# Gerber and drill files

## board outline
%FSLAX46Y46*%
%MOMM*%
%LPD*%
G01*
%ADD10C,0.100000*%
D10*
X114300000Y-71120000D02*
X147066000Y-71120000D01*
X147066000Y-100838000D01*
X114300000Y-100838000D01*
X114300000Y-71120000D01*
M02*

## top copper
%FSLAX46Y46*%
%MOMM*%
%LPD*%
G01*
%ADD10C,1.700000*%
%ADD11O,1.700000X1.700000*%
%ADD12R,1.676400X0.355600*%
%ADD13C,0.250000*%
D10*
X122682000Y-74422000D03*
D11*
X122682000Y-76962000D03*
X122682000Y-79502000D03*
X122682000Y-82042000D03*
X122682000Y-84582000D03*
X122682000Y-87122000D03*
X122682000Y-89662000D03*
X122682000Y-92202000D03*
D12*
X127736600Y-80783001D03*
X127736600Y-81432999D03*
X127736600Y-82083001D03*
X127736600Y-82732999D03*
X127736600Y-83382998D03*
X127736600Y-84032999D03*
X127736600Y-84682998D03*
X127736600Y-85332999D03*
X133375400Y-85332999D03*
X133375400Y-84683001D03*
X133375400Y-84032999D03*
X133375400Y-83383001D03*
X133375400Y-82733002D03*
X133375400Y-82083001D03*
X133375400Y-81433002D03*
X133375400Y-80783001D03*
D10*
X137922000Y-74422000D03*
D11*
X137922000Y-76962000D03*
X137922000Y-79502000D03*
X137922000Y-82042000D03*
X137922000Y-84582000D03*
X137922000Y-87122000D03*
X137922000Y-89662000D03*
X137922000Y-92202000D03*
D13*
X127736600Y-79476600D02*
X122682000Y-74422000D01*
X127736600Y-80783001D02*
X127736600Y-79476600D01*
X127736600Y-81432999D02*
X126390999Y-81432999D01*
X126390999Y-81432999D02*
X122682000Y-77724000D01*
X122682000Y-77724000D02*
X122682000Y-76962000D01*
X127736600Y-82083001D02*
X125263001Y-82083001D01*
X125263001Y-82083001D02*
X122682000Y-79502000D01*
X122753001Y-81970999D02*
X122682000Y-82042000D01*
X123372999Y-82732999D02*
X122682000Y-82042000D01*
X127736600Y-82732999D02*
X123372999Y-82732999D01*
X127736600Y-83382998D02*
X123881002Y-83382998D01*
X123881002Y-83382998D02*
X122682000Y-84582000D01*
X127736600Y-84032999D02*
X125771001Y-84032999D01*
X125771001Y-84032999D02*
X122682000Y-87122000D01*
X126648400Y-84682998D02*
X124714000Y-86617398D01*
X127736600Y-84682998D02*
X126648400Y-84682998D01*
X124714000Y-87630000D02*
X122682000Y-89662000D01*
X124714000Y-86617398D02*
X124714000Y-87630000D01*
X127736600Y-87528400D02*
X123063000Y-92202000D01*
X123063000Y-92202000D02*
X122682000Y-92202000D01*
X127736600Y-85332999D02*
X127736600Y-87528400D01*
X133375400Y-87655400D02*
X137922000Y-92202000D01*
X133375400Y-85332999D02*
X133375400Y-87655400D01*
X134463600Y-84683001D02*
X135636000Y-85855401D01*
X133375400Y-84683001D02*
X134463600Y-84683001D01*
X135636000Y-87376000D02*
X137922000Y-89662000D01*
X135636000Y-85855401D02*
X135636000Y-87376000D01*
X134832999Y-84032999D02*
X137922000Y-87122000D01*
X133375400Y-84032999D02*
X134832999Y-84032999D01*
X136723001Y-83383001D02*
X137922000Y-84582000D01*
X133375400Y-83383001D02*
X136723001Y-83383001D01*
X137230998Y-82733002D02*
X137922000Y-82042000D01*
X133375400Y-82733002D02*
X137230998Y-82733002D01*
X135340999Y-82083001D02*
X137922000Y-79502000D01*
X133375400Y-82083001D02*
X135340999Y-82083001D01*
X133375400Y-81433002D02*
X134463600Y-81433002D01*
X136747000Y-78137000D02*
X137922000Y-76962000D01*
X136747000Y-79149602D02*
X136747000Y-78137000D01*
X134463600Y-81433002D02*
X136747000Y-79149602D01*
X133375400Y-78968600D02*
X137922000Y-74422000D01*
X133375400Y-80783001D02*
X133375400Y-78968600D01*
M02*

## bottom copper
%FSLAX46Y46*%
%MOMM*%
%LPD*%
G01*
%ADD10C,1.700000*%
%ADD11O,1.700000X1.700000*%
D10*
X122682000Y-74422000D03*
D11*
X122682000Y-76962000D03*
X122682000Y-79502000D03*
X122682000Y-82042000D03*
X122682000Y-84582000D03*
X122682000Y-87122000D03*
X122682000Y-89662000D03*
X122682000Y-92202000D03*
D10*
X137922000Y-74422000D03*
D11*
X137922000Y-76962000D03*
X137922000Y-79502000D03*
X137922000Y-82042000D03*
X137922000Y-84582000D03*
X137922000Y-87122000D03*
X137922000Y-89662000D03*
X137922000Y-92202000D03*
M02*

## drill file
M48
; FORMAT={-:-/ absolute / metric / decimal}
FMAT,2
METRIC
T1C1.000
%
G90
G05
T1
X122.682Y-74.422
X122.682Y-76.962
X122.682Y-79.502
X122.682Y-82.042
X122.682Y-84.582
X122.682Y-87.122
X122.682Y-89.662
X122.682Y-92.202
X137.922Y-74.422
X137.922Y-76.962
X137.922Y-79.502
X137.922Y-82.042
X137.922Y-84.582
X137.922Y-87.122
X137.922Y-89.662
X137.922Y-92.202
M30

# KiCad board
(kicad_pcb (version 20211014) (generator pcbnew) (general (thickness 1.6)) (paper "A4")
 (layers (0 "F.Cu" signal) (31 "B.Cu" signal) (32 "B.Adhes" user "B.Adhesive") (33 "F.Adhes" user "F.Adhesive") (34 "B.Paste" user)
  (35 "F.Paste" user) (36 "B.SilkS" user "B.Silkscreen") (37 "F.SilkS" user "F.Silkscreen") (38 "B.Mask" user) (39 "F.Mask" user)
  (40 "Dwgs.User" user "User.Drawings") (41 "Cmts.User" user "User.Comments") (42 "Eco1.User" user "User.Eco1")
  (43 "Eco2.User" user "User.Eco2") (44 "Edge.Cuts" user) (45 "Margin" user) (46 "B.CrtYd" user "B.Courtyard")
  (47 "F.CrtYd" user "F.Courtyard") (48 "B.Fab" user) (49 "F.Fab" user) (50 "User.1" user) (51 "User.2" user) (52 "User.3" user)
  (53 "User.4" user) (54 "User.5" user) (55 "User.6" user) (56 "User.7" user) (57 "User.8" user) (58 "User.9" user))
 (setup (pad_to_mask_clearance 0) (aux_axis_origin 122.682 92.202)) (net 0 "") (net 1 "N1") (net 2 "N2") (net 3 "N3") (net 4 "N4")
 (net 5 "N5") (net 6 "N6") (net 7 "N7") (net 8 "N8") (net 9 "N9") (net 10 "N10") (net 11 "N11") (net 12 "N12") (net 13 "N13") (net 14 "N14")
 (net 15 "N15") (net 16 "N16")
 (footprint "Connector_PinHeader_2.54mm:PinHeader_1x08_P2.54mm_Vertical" (layer "F.Cu") (at 122.682 74.422)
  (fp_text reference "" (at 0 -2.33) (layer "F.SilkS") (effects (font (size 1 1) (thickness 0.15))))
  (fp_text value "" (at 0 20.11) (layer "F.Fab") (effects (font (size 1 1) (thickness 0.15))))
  (pad "1" thru_hole circle (at 0 0) (size 1.7 1.7) (drill 1) (layers *.Cu *.Mask) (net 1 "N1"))
  (pad "2" thru_hole oval (at 0 2.54) (size 1.7 1.7) (drill 1) (layers *.Cu *.Mask) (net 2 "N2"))
  (pad "3" thru_hole oval (at 0 5.08) (size 1.7 1.7) (drill 1) (layers *.Cu *.Mask) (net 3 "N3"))
  (pad "4" thru_hole oval (at 0 7.62) (size 1.7 1.7) (drill 1) (layers *.Cu *.Mask) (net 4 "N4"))
  (pad "5" thru_hole oval (at 0 10.16) (size 1.7 1.7) (drill 1) (layers *.Cu *.Mask) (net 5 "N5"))
  (pad "6" thru_hole oval (at 0 12.7) (size 1.7 1.7) (drill 1) (layers *.Cu *.Mask) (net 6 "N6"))
  (pad "7" thru_hole oval (at 0 15.24) (size 1.7 1.7) (drill 1) (layers *.Cu *.Mask) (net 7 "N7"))
  (pad "8" thru_hole oval (at 0 17.78) (size 1.7 1.7) (drill 1) (layers *.Cu *.Mask) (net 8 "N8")))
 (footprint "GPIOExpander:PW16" (layer "F.Cu") (at 130.556 83.058)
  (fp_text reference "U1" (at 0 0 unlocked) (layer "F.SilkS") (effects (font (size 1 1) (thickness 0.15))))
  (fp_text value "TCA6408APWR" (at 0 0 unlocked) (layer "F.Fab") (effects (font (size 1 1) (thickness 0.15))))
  (pad "1" smd rect (at -2.8194 -2.274999) (size 1.6764 0.3556) (layers "F.Cu" "F.Paste" "F.Mask") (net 1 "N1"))
  (pad "2" smd rect (at -2.8194 -1.625001) (size 1.6764 0.3556) (layers "F.Cu" "F.Paste" "F.Mask") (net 2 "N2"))
  (pad "3" smd rect (at -2.8194 -0.974999) (size 1.6764 0.3556) (layers "F.Cu" "F.Paste" "F.Mask") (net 3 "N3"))
  (pad "4" smd rect (at -2.8194 -0.325001) (size 1.6764 0.3556) (layers "F.Cu" "F.Paste" "F.Mask") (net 4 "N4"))
  (pad "5" smd rect (at -2.8194 0.324998) (size 1.6764 0.3556) (layers "F.Cu" "F.Paste" "F.Mask") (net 5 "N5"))
  (pad "6" smd rect (at -2.8194 0.974999) (size 1.6764 0.3556) (layers "F.Cu" "F.Paste" "F.Mask") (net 6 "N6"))
  (pad "7" smd rect (at -2.8194 1.624998) (size 1.6764 0.3556) (layers "F.Cu" "F.Paste" "F.Mask") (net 7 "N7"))
  (pad "8" smd rect (at -2.8194 2.274999) (size 1.6764 0.3556) (layers "F.Cu" "F.Paste" "F.Mask") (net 8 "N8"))
  (pad "9" smd rect (at 2.8194 2.274999) (size 1.6764 0.3556) (layers "F.Cu" "F.Paste" "F.Mask") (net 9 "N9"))
  (pad "10" smd rect (at 2.8194 1.625001) (size 1.6764 0.3556) (layers "F.Cu" "F.Paste" "F.Mask") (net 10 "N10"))
  (pad "11" smd rect (at 2.8194 0.974999) (size 1.6764 0.3556) (layers "F.Cu" "F.Paste" "F.Mask") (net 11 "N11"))
  (pad "12" smd rect (at 2.8194 0.325001) (size 1.6764 0.3556) (layers "F.Cu" "F.Paste" "F.Mask") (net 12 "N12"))
  (pad "13" smd rect (at 2.8194 -0.324998) (size 1.6764 0.3556) (layers "F.Cu" "F.Paste" "F.Mask") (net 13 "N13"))
  (pad "14" smd rect (at 2.8194 -0.974999) (size 1.6764 0.3556) (layers "F.Cu" "F.Paste" "F.Mask") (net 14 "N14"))
  (pad "15" smd rect (at 2.8194 -1.624998) (size 1.6764 0.3556) (layers "F.Cu" "F.Paste" "F.Mask") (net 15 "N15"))
  (pad "16" smd rect (at 2.8194 -2.274999) (size 1.6764 0.3556) (layers "F.Cu" "F.Paste" "F.Mask") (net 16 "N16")))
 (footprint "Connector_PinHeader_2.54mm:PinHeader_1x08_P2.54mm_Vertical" (layer "F.Cu") (at 137.922 74.422)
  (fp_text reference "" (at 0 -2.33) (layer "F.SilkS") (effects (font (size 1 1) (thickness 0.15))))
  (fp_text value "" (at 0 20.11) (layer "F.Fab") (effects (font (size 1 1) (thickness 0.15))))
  (pad "1" thru_hole circle (at 0 0) (size 1.7 1.7) (drill 1) (layers *.Cu *.Mask) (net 16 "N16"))
  (pad "2" thru_hole oval (at 0 2.54) (size 1.7 1.7) (drill 1) (layers *.Cu *.Mask) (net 15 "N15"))
  (pad "3" thru_hole oval (at 0 5.08) (size 1.7 1.7) (drill 1) (layers *.Cu *.Mask) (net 14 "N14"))
  (pad "4" thru_hole oval (at 0 7.62) (size 1.7 1.7) (drill 1) (layers *.Cu *.Mask) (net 13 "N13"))
  (pad "5" thru_hole oval (at 0 10.16) (size 1.7 1.7) (drill 1) (layers *.Cu *.Mask) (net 12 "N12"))
  (pad "6" thru_hole oval (at 0 12.7) (size 1.7 1.7) (drill 1) (layers *.Cu *.Mask) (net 11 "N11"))
  (pad "7" thru_hole oval (at 0 15.24) (size 1.7 1.7) (drill 1) (layers *.Cu *.Mask) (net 10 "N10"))
  (pad "8" thru_hole oval (at 0 17.78) (size 1.7 1.7) (drill 1) (layers *.Cu *.Mask) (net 9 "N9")))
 (gr_rect (start 114.3 71.12) (end 147.066 100.838) (layer "Edge.Cuts") (width 0.1) (fill none))
 (segment (start 127.7366 79.4766) (end 122.682 74.422) (width 0.25) (layer "F.Cu") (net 1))
 (segment (start 127.7366 80.783001) (end 127.7366 79.4766) (width 0.25) (layer "F.Cu") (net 1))
 (segment (start 127.7366 81.432999) (end 126.390999 81.432999) (width 0.25) (layer "F.Cu") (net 2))
 (segment (start 126.390999 81.432999) (end 122.682 77.724) (width 0.25) (layer "F.Cu") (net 2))
 (segment (start 122.682 77.724) (end 122.682 76.962) (width 0.25) (layer "F.Cu") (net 2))
 (segment (start 127.7366 82.083001) (end 125.263001 82.083001) (width 0.25) (layer "F.Cu") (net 3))
 (segment (start 125.263001 82.083001) (end 122.682 79.502) (width 0.25) (layer "F.Cu") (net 3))
 (segment (start 122.753001 81.970999) (end 122.682 82.042) (width 0.25) (layer "F.Cu") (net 4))
 (segment (start 123.372999 82.732999) (end 122.682 82.042) (width 0.25) (layer "F.Cu") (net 4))
 (segment (start 127.7366 82.732999) (end 123.372999 82.732999) (width 0.25) (layer "F.Cu") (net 4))
 (segment (start 127.7366 83.382998) (end 123.881002 83.382998) (width 0.25) (layer "F.Cu") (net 5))
 (segment (start 123.881002 83.382998) (end 122.682 84.582) (width 0.25) (layer "F.Cu") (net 5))
 (segment (start 127.7366 84.032999) (end 125.771001 84.032999) (width 0.25) (layer "F.Cu") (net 6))
 (segment (start 125.771001 84.032999) (end 122.682 87.122) (width 0.25) (layer "F.Cu") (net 6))
 (segment (start 126.6484 84.682998) (end 124.714 86.617398) (width 0.25) (layer "F.Cu") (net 7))
 (segment (start 127.7366 84.682998) (end 126.6484 84.682998) (width 0.25) (layer "F.Cu") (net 7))
 (segment (start 124.714 87.63) (end 122.682 89.662) (width 0.25) (layer "F.Cu") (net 7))
 (segment (start 124.714 86.617398) (end 124.714 87.63) (width 0.25) (layer "F.Cu") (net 7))
 (segment (start 127.7366 87.5284) (end 123.063 92.202) (width 0.25) (layer "F.Cu") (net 8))
 (segment (start 123.063 92.202) (end 122.682 92.202) (width 0.25) (layer "F.Cu") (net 8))
 (segment (start 127.7366 85.332999) (end 127.7366 87.5284) (width 0.25) (layer "F.Cu") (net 8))
 (segment (start 133.3754 87.6554) (end 137.922 92.202) (width 0.25) (layer "F.Cu") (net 9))
 (segment (start 133.3754 85.332999) (end 133.3754 87.6554) (width 0.25) (layer "F.Cu") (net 9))
 (segment (start 134.4636 84.683001) (end 135.636 85.855401) (width 0.25) (layer "F.Cu") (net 10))
 (segment (start 133.3754 84.683001) (end 134.4636 84.683001) (width 0.25) (layer "F.Cu") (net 10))
 (segment (start 135.636 87.376) (end 137.922 89.662) (width 0.25) (layer "F.Cu") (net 10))
 (segment (start 135.636 85.855401) (end 135.636 87.376) (width 0.25) (layer "F.Cu") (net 10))
 (segment (start 134.832999 84.032999) (end 137.922 87.122) (width 0.25) (layer "F.Cu") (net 11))
 (segment (start 133.3754 84.032999) (end 134.832999 84.032999) (width 0.25) (layer "F.Cu") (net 11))
 (segment (start 136.723001 83.383001) (end 137.922 84.582) (width 0.25) (layer "F.Cu") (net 12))
 (segment (start 133.3754 83.383001) (end 136.723001 83.383001) (width 0.25) (layer "F.Cu") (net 12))
 (segment (start 137.230998 82.733002) (end 137.922 82.042) (width 0.25) (layer "F.Cu") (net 13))
 (segment (start 133.3754 82.733002) (end 137.230998 82.733002) (width 0.25) (layer "F.Cu") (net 13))
 (segment (start 135.340999 82.083001) (end 137.922 79.502) (width 0.25) (layer "F.Cu") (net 14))
 (segment (start 133.3754 82.083001) (end 135.340999 82.083001) (width 0.25) (layer "F.Cu") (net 14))
 (segment (start 133.3754 81.433002) (end 134.4636 81.433002) (width 0.25) (layer "F.Cu") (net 15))
 (segment (start 136.747 78.137) (end 137.922 76.962) (width 0.25) (layer "F.Cu") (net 15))
 (segment (start 136.747 79.149602) (end 136.747 78.137) (width 0.25) (layer "F.Cu") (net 15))
 (segment (start 134.4636 81.433002) (end 136.747 79.149602) (width 0.25) (layer "F.Cu") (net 15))
 (segment (start 133.3754 78.9686) (end 137.922 74.422) (width 0.25) (layer "F.Cu") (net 16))
 (segment (start 133.3754 80.783001) (end 133.3754 78.9686) (width 0.25) (layer "F.Cu") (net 16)))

